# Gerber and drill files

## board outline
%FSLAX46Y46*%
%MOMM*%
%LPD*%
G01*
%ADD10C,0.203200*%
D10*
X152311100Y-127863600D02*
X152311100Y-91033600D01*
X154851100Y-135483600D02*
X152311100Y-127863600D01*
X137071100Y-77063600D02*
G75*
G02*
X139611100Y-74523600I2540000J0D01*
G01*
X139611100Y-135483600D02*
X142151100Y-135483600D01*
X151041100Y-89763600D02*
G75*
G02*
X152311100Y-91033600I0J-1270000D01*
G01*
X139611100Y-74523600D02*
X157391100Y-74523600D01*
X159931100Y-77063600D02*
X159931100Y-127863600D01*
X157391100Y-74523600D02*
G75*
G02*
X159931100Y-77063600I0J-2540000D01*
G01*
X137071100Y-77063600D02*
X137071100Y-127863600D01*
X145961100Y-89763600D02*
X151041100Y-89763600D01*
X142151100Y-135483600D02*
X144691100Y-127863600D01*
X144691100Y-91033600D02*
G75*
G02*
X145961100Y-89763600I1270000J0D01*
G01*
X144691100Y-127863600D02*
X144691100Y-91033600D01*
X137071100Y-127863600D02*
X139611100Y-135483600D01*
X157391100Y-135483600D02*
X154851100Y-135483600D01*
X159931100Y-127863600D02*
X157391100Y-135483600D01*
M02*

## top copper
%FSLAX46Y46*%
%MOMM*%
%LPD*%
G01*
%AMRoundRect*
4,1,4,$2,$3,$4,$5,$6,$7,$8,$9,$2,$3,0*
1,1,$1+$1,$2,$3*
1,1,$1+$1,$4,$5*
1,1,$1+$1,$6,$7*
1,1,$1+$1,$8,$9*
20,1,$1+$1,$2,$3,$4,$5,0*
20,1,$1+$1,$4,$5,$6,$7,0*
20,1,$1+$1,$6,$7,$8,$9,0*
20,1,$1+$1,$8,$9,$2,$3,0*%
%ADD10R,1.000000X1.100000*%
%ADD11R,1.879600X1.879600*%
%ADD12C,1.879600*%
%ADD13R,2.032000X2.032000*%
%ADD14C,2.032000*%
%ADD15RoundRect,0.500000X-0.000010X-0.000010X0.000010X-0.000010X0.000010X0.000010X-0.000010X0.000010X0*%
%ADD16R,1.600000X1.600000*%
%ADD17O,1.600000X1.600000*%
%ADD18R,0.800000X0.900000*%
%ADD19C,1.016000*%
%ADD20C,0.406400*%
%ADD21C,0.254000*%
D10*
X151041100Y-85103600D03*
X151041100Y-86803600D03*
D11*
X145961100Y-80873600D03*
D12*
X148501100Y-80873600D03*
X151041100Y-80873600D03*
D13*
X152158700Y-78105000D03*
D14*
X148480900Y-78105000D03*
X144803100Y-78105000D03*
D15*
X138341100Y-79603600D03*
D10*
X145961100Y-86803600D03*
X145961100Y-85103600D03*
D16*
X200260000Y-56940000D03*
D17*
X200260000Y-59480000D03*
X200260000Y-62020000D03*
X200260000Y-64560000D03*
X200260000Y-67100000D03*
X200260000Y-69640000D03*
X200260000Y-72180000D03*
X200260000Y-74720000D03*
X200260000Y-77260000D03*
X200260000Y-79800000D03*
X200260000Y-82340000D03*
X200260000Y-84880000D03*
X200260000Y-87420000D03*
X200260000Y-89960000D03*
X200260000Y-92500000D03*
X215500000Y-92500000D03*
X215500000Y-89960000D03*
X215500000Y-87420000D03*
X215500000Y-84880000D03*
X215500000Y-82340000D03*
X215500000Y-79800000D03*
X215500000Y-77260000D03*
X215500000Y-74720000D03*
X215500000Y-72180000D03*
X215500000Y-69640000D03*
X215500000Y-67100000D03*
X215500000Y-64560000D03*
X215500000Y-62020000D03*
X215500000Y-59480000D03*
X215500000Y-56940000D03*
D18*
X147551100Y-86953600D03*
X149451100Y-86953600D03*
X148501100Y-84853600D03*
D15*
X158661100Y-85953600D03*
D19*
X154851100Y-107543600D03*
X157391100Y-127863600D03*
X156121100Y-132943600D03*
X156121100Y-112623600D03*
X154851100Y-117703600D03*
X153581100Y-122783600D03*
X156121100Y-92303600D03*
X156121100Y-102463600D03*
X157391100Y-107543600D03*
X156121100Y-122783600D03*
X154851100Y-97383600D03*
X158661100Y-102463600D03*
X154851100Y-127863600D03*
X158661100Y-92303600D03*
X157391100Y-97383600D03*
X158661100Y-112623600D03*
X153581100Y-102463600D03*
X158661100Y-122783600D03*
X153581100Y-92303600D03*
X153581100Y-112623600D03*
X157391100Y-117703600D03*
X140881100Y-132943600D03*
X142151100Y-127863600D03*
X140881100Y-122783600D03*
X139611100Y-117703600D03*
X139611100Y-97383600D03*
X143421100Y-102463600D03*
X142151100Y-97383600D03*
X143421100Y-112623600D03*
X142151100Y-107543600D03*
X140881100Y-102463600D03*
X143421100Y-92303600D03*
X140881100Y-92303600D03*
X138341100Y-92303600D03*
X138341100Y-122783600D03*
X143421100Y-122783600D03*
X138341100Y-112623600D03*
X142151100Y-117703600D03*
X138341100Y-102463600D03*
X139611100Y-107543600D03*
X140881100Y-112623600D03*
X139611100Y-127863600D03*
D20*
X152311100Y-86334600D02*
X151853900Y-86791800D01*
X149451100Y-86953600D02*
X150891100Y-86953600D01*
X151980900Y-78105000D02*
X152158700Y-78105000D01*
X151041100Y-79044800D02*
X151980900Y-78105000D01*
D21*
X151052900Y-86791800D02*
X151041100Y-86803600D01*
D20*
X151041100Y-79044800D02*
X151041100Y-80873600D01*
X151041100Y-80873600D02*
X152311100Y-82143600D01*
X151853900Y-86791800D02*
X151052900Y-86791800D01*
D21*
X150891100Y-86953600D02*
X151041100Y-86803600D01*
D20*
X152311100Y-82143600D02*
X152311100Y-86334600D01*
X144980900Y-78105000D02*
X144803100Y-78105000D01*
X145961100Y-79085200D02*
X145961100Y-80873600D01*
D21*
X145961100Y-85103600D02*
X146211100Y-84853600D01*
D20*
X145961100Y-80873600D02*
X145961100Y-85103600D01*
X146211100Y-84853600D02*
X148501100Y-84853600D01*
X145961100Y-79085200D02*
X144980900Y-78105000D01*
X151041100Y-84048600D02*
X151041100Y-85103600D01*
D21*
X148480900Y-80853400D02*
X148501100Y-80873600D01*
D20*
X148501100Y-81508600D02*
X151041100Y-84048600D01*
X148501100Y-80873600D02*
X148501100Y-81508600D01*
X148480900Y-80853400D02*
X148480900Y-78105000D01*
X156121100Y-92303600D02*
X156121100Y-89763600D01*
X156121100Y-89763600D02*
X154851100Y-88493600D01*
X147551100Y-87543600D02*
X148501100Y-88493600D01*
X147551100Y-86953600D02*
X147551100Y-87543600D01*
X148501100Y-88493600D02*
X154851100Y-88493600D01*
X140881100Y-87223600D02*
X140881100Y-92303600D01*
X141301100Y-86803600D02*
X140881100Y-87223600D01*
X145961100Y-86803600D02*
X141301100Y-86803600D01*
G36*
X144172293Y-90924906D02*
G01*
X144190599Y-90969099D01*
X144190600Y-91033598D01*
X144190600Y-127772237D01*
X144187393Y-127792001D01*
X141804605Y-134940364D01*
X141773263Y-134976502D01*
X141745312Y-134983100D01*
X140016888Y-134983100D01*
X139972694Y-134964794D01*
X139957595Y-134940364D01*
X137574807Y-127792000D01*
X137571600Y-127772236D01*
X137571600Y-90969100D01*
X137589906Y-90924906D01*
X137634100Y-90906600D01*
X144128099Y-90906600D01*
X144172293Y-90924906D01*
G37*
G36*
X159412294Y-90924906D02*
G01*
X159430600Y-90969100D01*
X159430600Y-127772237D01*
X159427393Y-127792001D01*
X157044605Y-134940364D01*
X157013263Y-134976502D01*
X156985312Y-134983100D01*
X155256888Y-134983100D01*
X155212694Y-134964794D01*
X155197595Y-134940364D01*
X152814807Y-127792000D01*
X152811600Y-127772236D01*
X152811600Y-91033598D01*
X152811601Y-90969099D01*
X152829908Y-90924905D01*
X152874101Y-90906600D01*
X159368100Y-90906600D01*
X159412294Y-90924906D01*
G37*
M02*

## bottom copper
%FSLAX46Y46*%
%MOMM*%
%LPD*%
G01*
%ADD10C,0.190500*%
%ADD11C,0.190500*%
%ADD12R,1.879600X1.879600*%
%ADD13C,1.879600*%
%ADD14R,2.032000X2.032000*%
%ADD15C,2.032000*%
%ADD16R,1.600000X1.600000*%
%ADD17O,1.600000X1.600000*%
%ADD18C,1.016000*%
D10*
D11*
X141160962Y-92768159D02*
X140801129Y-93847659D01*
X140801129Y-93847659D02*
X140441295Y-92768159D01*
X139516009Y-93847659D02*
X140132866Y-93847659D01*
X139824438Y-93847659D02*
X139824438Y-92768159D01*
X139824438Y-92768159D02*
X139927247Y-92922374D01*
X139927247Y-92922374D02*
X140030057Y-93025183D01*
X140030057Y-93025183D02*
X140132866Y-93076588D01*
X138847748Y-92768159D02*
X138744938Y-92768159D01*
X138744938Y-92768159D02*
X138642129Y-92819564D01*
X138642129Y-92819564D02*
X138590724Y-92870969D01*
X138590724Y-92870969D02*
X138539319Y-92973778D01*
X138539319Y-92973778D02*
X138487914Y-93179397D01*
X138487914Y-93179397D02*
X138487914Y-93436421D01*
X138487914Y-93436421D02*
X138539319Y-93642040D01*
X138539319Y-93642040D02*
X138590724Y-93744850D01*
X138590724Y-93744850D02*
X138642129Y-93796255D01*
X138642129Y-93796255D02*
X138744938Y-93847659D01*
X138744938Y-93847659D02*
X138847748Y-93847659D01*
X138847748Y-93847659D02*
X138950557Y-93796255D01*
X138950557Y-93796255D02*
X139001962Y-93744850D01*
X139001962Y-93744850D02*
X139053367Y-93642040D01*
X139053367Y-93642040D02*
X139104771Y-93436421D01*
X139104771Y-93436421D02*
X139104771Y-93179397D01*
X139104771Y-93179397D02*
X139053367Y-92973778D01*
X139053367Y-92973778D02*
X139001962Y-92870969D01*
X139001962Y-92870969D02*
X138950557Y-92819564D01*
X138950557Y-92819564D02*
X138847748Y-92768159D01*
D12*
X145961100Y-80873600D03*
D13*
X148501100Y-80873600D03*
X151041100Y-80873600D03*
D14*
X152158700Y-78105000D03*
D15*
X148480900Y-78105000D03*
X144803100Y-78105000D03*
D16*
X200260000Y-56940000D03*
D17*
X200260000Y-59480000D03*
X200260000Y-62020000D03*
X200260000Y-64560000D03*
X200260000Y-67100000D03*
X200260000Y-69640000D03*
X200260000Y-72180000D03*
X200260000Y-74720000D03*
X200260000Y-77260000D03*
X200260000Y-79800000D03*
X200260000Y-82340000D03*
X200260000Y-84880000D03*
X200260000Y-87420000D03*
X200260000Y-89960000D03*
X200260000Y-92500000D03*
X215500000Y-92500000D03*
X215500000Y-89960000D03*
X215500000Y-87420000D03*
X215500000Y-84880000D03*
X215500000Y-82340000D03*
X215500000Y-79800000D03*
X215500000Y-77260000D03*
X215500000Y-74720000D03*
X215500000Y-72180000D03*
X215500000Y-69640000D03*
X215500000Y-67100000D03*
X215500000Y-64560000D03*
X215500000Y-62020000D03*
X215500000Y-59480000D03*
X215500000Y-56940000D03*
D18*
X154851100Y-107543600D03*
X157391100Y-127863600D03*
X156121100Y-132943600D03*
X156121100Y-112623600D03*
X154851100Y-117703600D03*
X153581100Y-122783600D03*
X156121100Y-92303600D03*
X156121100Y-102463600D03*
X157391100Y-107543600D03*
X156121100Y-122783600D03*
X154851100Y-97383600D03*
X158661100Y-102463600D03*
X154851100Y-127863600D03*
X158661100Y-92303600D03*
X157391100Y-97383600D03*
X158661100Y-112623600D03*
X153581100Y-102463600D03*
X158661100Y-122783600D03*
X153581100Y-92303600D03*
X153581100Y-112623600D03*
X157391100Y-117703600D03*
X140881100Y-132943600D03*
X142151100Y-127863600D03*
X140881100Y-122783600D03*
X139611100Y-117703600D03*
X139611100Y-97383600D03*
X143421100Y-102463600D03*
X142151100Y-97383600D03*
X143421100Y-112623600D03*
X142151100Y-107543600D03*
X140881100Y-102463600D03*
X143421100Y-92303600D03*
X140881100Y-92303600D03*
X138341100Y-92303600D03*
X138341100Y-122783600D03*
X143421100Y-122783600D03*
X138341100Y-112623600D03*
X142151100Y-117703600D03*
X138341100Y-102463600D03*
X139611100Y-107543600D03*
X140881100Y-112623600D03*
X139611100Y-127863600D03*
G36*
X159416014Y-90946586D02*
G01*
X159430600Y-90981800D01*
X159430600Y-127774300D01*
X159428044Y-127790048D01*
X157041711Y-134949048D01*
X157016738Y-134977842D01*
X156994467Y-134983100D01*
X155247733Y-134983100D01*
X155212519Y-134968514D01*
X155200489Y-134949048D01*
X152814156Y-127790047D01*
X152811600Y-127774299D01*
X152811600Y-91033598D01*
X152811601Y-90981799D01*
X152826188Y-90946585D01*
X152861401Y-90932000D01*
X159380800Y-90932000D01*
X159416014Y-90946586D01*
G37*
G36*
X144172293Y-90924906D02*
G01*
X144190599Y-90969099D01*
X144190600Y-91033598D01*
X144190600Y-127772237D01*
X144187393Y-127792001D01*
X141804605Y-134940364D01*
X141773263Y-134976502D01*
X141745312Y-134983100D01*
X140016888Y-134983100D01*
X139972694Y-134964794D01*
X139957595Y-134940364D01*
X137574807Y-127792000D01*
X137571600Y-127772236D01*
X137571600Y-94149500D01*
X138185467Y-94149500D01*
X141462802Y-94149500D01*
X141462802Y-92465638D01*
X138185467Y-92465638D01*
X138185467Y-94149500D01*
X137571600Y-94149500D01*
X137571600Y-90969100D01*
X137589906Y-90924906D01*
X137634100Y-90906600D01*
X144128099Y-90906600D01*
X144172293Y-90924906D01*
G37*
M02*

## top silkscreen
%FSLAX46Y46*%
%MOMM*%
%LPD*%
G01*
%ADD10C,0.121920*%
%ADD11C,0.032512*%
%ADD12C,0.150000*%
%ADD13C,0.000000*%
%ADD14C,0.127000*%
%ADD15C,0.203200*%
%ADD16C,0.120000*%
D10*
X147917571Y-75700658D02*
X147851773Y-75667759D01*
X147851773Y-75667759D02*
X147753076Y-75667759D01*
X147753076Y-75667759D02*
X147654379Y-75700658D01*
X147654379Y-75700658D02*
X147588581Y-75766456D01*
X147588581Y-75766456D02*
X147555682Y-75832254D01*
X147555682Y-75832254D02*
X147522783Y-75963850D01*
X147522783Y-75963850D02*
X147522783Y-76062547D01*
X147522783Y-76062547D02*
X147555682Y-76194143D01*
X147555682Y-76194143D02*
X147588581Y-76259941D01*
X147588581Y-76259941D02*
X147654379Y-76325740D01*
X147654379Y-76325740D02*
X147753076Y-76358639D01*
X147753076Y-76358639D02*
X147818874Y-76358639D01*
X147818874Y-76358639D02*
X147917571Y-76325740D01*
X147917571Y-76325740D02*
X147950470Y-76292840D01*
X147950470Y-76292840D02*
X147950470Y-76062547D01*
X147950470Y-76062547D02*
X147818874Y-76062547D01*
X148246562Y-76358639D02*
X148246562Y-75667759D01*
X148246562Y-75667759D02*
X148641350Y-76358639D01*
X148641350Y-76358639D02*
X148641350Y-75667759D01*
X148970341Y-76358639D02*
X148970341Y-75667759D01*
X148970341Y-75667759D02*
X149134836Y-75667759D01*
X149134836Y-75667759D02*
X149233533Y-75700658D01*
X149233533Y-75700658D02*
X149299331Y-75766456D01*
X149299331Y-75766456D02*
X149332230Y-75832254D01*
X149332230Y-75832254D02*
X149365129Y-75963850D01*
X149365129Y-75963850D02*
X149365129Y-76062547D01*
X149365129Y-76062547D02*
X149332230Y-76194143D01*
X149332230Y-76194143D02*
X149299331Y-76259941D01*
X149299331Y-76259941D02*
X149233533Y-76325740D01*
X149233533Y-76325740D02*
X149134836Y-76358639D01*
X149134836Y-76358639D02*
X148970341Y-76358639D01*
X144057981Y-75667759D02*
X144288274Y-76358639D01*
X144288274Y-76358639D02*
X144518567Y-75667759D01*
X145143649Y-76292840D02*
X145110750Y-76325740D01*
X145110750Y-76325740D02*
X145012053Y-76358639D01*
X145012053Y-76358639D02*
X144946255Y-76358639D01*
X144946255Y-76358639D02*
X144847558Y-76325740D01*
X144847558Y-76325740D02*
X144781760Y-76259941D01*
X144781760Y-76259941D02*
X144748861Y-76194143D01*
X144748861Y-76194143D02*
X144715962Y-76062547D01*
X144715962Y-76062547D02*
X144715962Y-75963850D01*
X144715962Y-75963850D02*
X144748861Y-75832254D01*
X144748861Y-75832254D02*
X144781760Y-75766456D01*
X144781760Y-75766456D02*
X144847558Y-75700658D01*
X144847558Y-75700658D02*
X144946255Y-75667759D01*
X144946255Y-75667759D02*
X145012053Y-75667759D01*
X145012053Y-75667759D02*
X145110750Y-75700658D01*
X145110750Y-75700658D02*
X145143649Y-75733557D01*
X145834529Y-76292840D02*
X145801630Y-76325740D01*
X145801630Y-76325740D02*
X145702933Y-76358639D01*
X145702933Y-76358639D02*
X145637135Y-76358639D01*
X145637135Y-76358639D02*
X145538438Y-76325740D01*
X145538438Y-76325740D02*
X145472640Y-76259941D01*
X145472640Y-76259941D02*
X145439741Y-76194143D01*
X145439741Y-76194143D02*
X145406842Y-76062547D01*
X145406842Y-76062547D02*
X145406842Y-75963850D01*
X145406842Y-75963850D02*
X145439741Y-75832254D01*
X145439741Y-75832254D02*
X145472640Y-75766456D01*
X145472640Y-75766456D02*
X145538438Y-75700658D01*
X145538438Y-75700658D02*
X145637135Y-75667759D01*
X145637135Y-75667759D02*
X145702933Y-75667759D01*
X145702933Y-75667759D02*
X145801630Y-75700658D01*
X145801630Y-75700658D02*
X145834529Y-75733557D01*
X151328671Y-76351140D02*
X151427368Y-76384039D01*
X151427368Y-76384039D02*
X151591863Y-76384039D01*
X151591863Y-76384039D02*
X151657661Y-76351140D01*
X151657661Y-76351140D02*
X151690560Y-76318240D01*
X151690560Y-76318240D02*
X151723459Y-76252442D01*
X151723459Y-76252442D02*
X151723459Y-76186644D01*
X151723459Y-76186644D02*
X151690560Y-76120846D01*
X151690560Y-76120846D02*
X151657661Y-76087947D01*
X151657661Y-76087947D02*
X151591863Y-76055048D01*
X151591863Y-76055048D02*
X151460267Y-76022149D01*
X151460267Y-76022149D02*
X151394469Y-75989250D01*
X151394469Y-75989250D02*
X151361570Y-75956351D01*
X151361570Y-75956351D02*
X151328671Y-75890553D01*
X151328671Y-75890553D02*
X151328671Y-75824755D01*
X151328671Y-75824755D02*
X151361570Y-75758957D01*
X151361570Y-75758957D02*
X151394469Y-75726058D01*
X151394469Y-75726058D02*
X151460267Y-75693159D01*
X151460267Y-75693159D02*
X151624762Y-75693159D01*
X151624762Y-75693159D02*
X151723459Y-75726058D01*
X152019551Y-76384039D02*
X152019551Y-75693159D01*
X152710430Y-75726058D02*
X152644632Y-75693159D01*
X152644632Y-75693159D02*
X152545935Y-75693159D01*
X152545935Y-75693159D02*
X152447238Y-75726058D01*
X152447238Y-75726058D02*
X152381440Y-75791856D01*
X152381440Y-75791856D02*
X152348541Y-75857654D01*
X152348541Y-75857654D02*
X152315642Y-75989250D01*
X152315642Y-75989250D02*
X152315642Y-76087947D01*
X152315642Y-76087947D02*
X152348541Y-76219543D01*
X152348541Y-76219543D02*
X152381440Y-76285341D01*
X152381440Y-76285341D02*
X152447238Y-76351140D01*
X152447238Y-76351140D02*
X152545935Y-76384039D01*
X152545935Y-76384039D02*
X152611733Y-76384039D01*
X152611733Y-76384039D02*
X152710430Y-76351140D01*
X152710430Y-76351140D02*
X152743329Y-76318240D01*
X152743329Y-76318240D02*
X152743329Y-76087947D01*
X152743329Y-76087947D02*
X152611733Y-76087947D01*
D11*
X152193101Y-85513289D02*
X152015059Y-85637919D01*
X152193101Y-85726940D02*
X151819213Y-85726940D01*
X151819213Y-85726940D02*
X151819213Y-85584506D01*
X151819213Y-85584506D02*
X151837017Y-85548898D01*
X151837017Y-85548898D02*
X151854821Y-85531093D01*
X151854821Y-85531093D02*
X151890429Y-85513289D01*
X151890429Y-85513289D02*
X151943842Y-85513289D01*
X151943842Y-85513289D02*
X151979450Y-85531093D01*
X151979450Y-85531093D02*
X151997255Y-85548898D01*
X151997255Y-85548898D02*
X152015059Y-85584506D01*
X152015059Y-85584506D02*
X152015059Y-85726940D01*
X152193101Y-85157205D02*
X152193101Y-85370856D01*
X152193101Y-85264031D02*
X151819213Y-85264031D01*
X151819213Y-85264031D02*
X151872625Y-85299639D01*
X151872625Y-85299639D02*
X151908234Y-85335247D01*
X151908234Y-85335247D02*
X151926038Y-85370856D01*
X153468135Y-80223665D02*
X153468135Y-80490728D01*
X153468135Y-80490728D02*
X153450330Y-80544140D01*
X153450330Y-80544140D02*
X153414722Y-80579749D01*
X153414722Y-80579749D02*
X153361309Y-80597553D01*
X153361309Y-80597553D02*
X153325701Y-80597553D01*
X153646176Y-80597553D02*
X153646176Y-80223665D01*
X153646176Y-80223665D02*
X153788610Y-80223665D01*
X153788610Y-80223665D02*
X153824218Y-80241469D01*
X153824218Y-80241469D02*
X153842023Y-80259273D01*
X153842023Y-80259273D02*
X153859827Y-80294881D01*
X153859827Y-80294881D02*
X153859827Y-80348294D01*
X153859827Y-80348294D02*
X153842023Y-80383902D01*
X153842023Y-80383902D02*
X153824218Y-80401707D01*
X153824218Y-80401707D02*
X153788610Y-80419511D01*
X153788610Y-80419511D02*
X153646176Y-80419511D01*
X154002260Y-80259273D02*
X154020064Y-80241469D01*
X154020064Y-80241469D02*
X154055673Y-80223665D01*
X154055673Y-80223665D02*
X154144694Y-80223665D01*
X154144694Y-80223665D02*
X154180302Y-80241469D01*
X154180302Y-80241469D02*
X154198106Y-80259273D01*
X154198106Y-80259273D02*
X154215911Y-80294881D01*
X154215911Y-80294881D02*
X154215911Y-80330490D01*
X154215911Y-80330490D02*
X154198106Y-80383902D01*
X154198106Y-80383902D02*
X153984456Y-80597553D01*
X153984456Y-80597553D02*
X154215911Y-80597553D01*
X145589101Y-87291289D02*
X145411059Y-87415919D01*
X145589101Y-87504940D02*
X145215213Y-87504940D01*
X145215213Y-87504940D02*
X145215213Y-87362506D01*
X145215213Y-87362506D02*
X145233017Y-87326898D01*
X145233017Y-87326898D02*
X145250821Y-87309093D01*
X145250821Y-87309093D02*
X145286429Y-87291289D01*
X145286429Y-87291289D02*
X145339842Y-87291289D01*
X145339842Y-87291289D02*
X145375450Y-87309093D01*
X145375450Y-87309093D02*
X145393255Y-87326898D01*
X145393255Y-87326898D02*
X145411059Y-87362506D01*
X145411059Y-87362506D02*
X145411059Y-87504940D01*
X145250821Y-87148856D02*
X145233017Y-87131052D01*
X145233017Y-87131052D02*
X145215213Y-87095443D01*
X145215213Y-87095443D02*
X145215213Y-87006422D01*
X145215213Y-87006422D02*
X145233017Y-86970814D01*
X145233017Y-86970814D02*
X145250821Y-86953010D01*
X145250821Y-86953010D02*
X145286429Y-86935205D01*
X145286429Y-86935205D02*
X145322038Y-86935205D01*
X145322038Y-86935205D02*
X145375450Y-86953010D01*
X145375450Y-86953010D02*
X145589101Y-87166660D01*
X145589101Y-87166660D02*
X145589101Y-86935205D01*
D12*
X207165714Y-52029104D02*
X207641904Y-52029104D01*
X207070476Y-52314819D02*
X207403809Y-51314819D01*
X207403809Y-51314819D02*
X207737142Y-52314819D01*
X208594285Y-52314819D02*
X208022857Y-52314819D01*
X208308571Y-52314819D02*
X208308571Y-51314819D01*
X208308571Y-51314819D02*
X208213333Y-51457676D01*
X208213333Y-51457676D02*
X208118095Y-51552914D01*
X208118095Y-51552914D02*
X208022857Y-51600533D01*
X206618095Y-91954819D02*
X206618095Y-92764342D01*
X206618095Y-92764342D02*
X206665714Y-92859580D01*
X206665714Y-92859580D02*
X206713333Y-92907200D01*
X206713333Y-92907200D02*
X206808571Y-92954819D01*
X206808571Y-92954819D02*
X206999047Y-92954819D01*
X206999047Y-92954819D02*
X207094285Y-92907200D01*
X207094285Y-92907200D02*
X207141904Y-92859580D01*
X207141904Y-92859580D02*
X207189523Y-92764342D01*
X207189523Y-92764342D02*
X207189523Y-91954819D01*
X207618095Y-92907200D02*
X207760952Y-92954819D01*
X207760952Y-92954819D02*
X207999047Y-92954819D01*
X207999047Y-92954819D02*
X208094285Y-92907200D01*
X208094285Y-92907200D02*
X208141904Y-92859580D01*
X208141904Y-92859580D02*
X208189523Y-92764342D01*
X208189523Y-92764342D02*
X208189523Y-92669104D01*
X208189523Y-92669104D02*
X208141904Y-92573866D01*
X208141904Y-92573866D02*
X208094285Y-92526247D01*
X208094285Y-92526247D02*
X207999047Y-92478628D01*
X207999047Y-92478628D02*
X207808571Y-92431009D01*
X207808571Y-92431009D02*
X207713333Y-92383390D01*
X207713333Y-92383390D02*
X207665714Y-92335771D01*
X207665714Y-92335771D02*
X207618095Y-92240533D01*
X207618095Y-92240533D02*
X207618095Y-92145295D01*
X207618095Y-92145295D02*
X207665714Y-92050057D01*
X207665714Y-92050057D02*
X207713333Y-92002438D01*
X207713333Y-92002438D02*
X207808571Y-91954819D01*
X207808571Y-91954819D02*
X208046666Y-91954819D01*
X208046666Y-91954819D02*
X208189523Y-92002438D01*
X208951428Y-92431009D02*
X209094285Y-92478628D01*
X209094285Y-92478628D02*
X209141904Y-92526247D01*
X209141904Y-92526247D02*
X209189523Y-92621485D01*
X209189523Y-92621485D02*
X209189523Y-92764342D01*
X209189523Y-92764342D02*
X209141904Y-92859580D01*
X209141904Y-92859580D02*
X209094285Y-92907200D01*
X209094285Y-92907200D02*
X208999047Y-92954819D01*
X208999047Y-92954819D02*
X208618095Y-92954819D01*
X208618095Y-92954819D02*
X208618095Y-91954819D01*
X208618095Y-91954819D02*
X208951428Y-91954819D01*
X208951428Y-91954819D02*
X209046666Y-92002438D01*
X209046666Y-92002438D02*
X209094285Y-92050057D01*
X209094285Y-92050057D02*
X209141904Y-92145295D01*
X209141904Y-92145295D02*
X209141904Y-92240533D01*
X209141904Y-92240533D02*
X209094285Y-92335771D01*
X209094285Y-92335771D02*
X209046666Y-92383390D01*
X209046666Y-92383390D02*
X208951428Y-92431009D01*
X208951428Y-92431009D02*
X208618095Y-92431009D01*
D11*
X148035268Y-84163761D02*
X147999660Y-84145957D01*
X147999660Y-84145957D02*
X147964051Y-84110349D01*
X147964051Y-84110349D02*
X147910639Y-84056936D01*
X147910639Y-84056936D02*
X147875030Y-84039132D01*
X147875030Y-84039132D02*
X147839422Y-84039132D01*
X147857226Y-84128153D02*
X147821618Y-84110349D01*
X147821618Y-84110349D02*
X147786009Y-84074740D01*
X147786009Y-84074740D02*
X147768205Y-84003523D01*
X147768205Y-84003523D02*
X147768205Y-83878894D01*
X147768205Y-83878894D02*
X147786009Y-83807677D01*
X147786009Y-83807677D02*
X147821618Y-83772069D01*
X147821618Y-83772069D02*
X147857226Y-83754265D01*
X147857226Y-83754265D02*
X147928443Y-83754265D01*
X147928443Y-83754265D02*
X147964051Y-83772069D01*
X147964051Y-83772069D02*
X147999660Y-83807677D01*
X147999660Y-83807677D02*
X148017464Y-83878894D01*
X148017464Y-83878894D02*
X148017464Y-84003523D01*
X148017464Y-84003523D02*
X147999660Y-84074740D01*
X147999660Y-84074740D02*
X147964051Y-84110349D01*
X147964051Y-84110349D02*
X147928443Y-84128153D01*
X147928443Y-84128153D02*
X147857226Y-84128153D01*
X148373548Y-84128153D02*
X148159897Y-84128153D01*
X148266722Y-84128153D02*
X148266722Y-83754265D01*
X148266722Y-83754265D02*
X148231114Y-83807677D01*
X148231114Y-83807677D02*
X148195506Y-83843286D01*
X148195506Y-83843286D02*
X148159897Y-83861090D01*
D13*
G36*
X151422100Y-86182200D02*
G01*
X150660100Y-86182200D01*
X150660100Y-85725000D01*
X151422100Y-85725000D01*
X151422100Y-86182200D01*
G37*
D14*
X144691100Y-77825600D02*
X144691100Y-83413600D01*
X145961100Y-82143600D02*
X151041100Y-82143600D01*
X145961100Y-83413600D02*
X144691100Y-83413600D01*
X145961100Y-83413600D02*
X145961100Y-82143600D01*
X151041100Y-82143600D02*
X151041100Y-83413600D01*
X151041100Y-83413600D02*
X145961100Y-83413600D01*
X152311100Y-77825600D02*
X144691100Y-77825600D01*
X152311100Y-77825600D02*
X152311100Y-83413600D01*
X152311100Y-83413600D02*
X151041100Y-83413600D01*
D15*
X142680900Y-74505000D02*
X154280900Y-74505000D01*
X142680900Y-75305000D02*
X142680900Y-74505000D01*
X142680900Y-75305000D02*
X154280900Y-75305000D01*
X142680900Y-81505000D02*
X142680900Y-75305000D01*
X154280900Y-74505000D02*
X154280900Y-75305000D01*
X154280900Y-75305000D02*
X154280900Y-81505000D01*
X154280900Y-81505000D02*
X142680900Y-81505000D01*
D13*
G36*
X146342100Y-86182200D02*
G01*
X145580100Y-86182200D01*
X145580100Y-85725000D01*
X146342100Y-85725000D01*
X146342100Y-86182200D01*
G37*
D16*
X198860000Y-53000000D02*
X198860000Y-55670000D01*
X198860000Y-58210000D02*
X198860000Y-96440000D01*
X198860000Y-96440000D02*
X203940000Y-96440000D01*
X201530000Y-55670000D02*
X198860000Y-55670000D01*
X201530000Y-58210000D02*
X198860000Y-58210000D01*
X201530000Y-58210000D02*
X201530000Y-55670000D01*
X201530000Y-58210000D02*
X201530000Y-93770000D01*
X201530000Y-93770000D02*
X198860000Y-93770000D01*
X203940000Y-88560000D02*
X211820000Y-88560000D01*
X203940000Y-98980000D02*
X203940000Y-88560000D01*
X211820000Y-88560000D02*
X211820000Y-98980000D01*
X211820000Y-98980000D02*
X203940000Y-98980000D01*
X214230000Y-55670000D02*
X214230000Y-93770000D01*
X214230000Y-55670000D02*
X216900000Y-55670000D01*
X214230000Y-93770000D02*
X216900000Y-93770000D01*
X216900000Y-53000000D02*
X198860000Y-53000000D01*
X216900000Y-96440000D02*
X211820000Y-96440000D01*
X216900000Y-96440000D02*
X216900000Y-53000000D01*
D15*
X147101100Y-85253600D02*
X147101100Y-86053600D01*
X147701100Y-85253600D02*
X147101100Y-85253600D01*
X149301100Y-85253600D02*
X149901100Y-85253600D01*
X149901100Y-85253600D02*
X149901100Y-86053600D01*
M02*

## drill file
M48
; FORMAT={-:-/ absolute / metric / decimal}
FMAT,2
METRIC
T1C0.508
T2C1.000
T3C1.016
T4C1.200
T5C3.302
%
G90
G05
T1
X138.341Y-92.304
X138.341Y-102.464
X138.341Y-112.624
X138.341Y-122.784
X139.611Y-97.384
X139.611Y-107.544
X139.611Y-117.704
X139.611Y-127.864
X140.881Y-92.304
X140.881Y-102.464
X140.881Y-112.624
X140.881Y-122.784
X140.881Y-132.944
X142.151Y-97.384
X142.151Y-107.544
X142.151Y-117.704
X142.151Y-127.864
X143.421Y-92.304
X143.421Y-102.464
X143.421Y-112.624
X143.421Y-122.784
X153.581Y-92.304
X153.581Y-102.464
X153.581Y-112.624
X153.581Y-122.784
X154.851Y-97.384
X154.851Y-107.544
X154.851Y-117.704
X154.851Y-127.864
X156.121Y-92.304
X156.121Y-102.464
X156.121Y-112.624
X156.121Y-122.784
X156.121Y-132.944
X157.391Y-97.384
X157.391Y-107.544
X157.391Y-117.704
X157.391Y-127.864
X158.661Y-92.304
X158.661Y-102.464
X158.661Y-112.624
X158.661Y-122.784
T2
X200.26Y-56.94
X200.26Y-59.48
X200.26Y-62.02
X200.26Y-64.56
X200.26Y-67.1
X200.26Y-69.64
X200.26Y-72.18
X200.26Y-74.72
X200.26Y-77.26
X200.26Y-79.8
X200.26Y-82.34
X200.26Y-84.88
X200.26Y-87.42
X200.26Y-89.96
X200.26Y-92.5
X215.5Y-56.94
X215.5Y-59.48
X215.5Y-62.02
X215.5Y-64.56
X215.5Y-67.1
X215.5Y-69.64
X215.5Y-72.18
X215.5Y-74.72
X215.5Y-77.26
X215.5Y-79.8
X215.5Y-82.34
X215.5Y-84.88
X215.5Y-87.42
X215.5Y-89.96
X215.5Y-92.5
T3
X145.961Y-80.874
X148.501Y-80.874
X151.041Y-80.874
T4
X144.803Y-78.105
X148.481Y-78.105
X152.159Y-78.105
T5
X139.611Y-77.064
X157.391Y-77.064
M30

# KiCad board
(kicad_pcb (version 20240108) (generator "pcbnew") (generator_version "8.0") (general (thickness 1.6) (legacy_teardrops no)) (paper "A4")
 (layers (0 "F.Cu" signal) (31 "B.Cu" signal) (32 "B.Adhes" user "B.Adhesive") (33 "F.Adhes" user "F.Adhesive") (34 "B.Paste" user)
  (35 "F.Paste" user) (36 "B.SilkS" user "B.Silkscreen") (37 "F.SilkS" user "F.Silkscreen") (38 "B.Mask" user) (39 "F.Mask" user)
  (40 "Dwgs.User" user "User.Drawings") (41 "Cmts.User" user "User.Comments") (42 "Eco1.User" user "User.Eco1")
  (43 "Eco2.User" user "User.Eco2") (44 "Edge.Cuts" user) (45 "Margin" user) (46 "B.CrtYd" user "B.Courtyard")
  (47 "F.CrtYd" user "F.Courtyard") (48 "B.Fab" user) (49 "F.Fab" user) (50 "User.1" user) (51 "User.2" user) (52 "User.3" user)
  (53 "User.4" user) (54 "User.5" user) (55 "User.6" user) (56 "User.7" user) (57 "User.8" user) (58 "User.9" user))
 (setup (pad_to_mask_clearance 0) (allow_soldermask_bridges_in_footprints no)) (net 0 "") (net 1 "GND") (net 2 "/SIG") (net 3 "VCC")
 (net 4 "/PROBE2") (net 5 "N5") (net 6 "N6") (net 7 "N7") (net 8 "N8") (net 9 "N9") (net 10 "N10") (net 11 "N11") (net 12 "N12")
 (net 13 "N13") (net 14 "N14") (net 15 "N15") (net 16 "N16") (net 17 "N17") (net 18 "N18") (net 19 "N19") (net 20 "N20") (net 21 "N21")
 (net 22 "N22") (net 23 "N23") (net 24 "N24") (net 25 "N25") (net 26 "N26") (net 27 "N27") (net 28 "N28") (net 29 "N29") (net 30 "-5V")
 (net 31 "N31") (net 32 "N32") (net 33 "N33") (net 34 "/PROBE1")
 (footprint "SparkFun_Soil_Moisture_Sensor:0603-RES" (layer "F.Cu") (at 151.0411 85.9536 -90)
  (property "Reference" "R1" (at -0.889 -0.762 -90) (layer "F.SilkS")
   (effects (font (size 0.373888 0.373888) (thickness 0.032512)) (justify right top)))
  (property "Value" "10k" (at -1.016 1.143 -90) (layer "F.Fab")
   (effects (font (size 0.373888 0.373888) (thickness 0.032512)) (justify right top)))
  (fp_poly
   (pts (xy -0.2286 0.381) (xy 0.2286 0.381) (xy 0.2286 -0.381) (xy -0.2286 -0.381)) (stroke (width 0) (type default)) (fill solid)
   (layer "F.SilkS"))
  (pad "1" smd rect (at -0.85 0 270) (size 1.1 1) (layers "F.Cu" "F.Paste" "F.Mask") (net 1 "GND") (solder_mask_margin 0.1016)
   (thermal_bridge_angle 0))
  (pad "2" smd rect (at 0.85 0 270) (size 1.1 1) (layers "F.Cu" "F.Paste" "F.Mask") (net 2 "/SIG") (solder_mask_margin 0.1016)
   (thermal_bridge_angle 0)))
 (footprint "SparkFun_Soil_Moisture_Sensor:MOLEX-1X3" (layer "F.Cu") (at 145.9611 80.8736)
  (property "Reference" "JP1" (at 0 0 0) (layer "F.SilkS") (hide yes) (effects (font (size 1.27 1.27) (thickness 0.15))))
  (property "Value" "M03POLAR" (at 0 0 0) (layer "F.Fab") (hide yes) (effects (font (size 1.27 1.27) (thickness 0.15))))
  (fp_line (start -1.27 -3.048) (end -1.27 2.54) (stroke (width 0.127) (type solid)) (layer "F.SilkS"))
  (fp_line (start 0 1.27) (end 5.08 1.27) (stroke (width 0.127) (type solid)) (layer "F.SilkS"))
  (fp_line (start 0 2.54) (end -1.27 2.54) (stroke (width 0.127) (type solid)) (layer "F.SilkS"))
  (fp_line (start 0 2.54) (end 0 1.27) (stroke (width 0.127) (type solid)) (layer "F.SilkS"))
  (fp_line (start 5.08 1.27) (end 5.08 2.54) (stroke (width 0.127) (type solid)) (layer "F.SilkS"))
  (fp_line (start 5.08 2.54) (end 0 2.54) (stroke (width 0.127) (type solid)) (layer "F.SilkS"))
  (fp_line (start 6.35 -3.048) (end -1.27 -3.048) (stroke (width 0.127) (type solid)) (layer "F.SilkS"))
  (fp_line (start 6.35 -3.048) (end 6.35 2.54) (stroke (width 0.127) (type solid)) (layer "F.SilkS"))
  (fp_line (start 6.35 2.54) (end 5.08 2.54) (stroke (width 0.127) (type solid)) (layer "F.SilkS"))
  (pad "1" thru_hole rect (at 0 0) (size 1.8796 1.8796) (drill 1.016) (layers "*.Cu" "*.Mask") (remove_unused_layers no) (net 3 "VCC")
   (solder_mask_margin 0.1016) (thermal_bridge_angle 0))
  (pad "2" thru_hole circle (at 2.54 0) (size 1.8796 1.8796) (drill 1.016) (layers "*.Cu" "*.Mask") (remove_unused_layers no) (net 1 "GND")
   (solder_mask_margin 0.1016) (thermal_bridge_angle 0))
  (pad "3" thru_hole circle (at 5.08 0) (size 1.8796 1.8796) (drill 1.016) (layers "*.Cu" "*.Mask") (remove_unused_layers no) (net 2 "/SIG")
   (solder_mask_margin 0.1016) (thermal_bridge_angle 0)))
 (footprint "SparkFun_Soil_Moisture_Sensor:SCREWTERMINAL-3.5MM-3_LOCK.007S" (layer "F.Cu") (at 151.9809 78.105 180)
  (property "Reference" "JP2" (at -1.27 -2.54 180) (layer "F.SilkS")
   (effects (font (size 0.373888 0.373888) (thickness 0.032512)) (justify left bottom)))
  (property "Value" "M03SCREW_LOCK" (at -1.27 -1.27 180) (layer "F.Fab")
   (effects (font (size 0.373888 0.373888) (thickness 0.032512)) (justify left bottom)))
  (fp_line (start 9.3 3.6) (end -2.3 3.6) (stroke (width 0.2032) (type solid)) (layer "F.SilkS"))
  (fp_line (start 9.3 2.8) (end 9.3 3.6) (stroke (width 0.2032) (type solid)) (layer "F.SilkS"))
  (fp_line (start 9.3 2.8) (end -2.3 2.8) (stroke (width 0.2032) (type solid)) (layer "F.SilkS"))
  (fp_line (start 9.3 -3.4) (end 9.3 2.8) (stroke (width 0.2032) (type solid)) (layer "F.SilkS"))
  (fp_line (start -2.3 3.6) (end -2.3 2.8) (stroke (width 0.2032) (type solid)) (layer "F.SilkS"))
  (fp_line (start -2.3 2.8) (end -2.3 -3.4) (stroke (width 0.2032) (type solid)) (layer "F.SilkS"))
  (fp_line (start -2.3 -3.4) (end 9.3 -3.4) (stroke (width 0.2032) (type solid)) (layer "F.SilkS"))
  (pad "1" thru_hole rect (at -0.1778 0 180) (size 2.032 2.032) (drill 1.2) (layers "*.Cu" "*.Mask") (remove_unused_layers no)
   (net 2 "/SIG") (solder_mask_margin 0.1016) (thermal_bridge_angle 0))
  (pad "2" thru_hole circle (at 3.5 0 180) (size 2.032 2.032) (drill 1.2) (layers "*.Cu" "*.Mask") (remove_unused_layers no) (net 1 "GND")
   (solder_mask_margin 0.1016) (thermal_bridge_angle 0))
  (pad "3" thru_hole circle (at 7.1778 0 180) (size 2.032 2.032) (drill 1.2) (layers "*.Cu" "*.Mask") (remove_unused_layers no)
   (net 3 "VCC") (solder_mask_margin 0.1016) (thermal_bridge_angle 0)))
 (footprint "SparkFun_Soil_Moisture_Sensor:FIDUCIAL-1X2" (layer "F.Cu") (at 138.3411 79.6036)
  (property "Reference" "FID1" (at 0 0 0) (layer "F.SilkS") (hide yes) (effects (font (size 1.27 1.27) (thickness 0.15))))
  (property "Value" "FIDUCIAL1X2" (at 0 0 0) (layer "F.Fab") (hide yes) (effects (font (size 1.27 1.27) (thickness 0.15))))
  (pad "1" smd roundrect (at 0 0) (size 1 1) (layers "F.Cu" "F.Mask") (roundrect_rratio 0.5) (solder_mask_margin 0.1016)
   (thermal_bridge_angle 0)))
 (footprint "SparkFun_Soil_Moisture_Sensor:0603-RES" (layer "F.Cu") (at 145.9611 85.9536 90)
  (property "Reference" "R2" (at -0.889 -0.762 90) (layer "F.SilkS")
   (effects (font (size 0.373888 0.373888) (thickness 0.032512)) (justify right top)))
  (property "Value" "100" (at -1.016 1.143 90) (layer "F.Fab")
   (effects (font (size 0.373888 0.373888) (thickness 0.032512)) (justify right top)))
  (fp_poly
   (pts (xy -0.2286 0.381) (xy 0.2286 0.381) (xy 0.2286 -0.381) (xy -0.2286 -0.381)) (stroke (width 0) (type default)) (fill solid)
   (layer "F.SilkS"))
  (pad "1" smd rect (at -0.85 0 90) (size 1.1 1) (layers "F.Cu" "F.Paste" "F.Mask") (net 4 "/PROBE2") (solder_mask_margin 0.1016)
   (thermal_bridge_angle 0))
  (pad "2" smd rect (at 0.85 0 90) (size 1.1 1) (layers "F.Cu" "F.Paste" "F.Mask") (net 3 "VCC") (solder_mask_margin 0.1016)
   (thermal_bridge_angle 0)))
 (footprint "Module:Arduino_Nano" (layer "F.Cu") (at 200.26 56.94)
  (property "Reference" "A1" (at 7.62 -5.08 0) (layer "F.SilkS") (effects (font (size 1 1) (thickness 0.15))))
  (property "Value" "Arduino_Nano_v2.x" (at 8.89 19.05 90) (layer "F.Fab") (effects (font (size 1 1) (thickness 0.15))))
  (fp_line (start -1.4 -3.94) (end -1.4 -1.27) (stroke (width 0.12) (type solid)) (layer "F.SilkS"))
  (fp_line (start -1.4 1.27) (end -1.4 39.5) (stroke (width 0.12) (type solid)) (layer "F.SilkS"))
  (fp_line (start -1.4 39.5) (end 3.68 39.5) (stroke (width 0.12) (type solid)) (layer "F.SilkS"))
  (fp_line (start 1.27 -1.27) (end -1.4 -1.27) (stroke (width 0.12) (type solid)) (layer "F.SilkS"))
  (fp_line (start 1.27 1.27) (end -1.4 1.27) (stroke (width 0.12) (type solid)) (layer "F.SilkS"))
  (fp_line (start 1.27 1.27) (end 1.27 -1.27) (stroke (width 0.12) (type solid)) (layer "F.SilkS"))
  (fp_line (start 1.27 1.27) (end 1.27 36.83) (stroke (width 0.12) (type solid)) (layer "F.SilkS"))
  (fp_line (start 1.27 36.83) (end -1.4 36.83) (stroke (width 0.12) (type solid)) (layer "F.SilkS"))
  (fp_line (start 3.68 31.62) (end 11.56 31.62) (stroke (width 0.12) (type solid)) (layer "F.SilkS"))
  (fp_line (start 3.68 42.04) (end 3.68 31.62) (stroke (width 0.12) (type solid)) (layer "F.SilkS"))
  (fp_line (start 11.56 31.62) (end 11.56 42.04) (stroke (width 0.12) (type solid)) (layer "F.SilkS"))
  (fp_line (start 11.56 42.04) (end 3.68 42.04) (stroke (width 0.12) (type solid)) (layer "F.SilkS"))
  (fp_line (start 13.97 -1.27) (end 13.97 36.83) (stroke (width 0.12) (type solid)) (layer "F.SilkS"))
  (fp_line (start 13.97 -1.27) (end 16.64 -1.27) (stroke (width 0.12) (type solid)) (layer "F.SilkS"))
  (fp_line (start 13.97 36.83) (end 16.64 36.83) (stroke (width 0.12) (type solid)) (layer "F.SilkS"))
  (fp_line (start 16.64 -3.94) (end -1.4 -3.94) (stroke (width 0.12) (type solid)) (layer "F.SilkS"))
  (fp_line (start 16.64 39.5) (end 11.56 39.5) (stroke (width 0.12) (type solid)) (layer "F.SilkS"))
  (fp_line (start 16.64 39.5) (end 16.64 -3.94) (stroke (width 0.12) (type solid)) (layer "F.SilkS"))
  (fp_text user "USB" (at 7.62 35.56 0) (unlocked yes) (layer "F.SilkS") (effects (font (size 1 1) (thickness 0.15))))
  (pad "1" thru_hole rect (at 0 0) (size 1.6 1.6) (drill 1) (layers "*.Cu" "*.Mask") (remove_unused_layers no) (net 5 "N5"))
  (pad "2" thru_hole oval (at 0 2.54) (size 1.6 1.6) (drill 1) (layers "*.Cu" "*.Mask") (remove_unused_layers no) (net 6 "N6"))
  (pad "3" thru_hole oval (at 0 5.08) (size 1.6 1.6) (drill 1) (layers "*.Cu" "*.Mask") (remove_unused_layers no) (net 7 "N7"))
  (pad "4" thru_hole oval (at 0 7.62) (size 1.6 1.6) (drill 1) (layers "*.Cu" "*.Mask") (remove_unused_layers no) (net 1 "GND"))
  (pad "5" thru_hole oval (at 0 10.16) (size 1.6 1.6) (drill 1) (layers "*.Cu" "*.Mask") (remove_unused_layers no) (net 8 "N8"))
  (pad "6" thru_hole oval (at 0 12.7) (size 1.6 1.6) (drill 1) (layers "*.Cu" "*.Mask") (remove_unused_layers no) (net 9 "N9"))
  (pad "7" thru_hole oval (at 0 15.24) (size 1.6 1.6) (drill 1) (layers "*.Cu" "*.Mask") (remove_unused_layers no) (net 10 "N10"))
  (pad "8" thru_hole oval (at 0 17.78) (size 1.6 1.6) (drill 1) (layers "*.Cu" "*.Mask") (remove_unused_layers no) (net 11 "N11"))
  (pad "9" thru_hole oval (at 0 20.32) (size 1.6 1.6) (drill 1) (layers "*.Cu" "*.Mask") (remove_unused_layers no) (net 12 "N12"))
  (pad "10" thru_hole oval (at 0 22.86) (size 1.6 1.6) (drill 1) (layers "*.Cu" "*.Mask") (remove_unused_layers no) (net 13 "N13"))
  (pad "11" thru_hole oval (at 0 25.4) (size 1.6 1.6) (drill 1) (layers "*.Cu" "*.Mask") (remove_unused_layers no) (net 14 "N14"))
  (pad "12" thru_hole oval (at 0 27.94) (size 1.6 1.6) (drill 1) (layers "*.Cu" "*.Mask") (remove_unused_layers no) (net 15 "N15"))
  (pad "13" thru_hole oval (at 0 30.48) (size 1.6 1.6) (drill 1) (layers "*.Cu" "*.Mask") (remove_unused_layers no) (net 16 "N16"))
  (pad "14" thru_hole oval (at 0 33.02) (size 1.6 1.6) (drill 1) (layers "*.Cu" "*.Mask") (remove_unused_layers no) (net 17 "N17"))
  (pad "15" thru_hole oval (at 0 35.56) (size 1.6 1.6) (drill 1) (layers "*.Cu" "*.Mask") (remove_unused_layers no) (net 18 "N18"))
  (pad "16" thru_hole oval (at 15.24 35.56) (size 1.6 1.6) (drill 1) (layers "*.Cu" "*.Mask") (remove_unused_layers no) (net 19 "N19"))
  (pad "17" thru_hole oval (at 15.24 33.02) (size 1.6 1.6) (drill 1) (layers "*.Cu" "*.Mask") (remove_unused_layers no) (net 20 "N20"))
  (pad "18" thru_hole oval (at 15.24 30.48) (size 1.6 1.6) (drill 1) (layers "*.Cu" "*.Mask") (remove_unused_layers no) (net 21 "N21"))
  (pad "19" thru_hole oval (at 15.24 27.94) (size 1.6 1.6) (drill 1) (layers "*.Cu" "*.Mask") (remove_unused_layers no) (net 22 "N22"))
  (pad "20" thru_hole oval (at 15.24 25.4) (size 1.6 1.6) (drill 1) (layers "*.Cu" "*.Mask") (remove_unused_layers no) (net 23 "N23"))
  (pad "21" thru_hole oval (at 15.24 22.86) (size 1.6 1.6) (drill 1) (layers "*.Cu" "*.Mask") (remove_unused_layers no) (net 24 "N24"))
  (pad "22" thru_hole oval (at 15.24 20.32) (size 1.6 1.6) (drill 1) (layers "*.Cu" "*.Mask") (remove_unused_layers no) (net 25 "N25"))
  (pad "23" thru_hole oval (at 15.24 17.78) (size 1.6 1.6) (drill 1) (layers "*.Cu" "*.Mask") (remove_unused_layers no) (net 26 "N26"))
  (pad "24" thru_hole oval (at 15.24 15.24) (size 1.6 1.6) (drill 1) (layers "*.Cu" "*.Mask") (remove_unused_layers no) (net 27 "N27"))
  (pad "25" thru_hole oval (at 15.24 12.7) (size 1.6 1.6) (drill 1) (layers "*.Cu" "*.Mask") (remove_unused_layers no) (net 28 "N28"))
  (pad "26" thru_hole oval (at 15.24 10.16) (size 1.6 1.6) (drill 1) (layers "*.Cu" "*.Mask") (remove_unused_layers no) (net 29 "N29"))
  (pad "27" thru_hole oval (at 15.24 7.62) (size 1.6 1.6) (drill 1) (layers "*.Cu" "*.Mask") (remove_unused_layers no) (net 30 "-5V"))
  (pad "28" thru_hole oval (at 15.24 5.08) (size 1.6 1.6) (drill 1) (layers "*.Cu" "*.Mask") (remove_unused_layers no) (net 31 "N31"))
  (pad "29" thru_hole oval (at 15.24 2.54) (size 1.6 1.6) (drill 1) (layers "*.Cu" "*.Mask") (remove_unused_layers no) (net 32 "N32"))
  (pad "30" thru_hole oval (at 15.24 0) (size 1.6 1.6) (drill 1) (layers "*.Cu" "*.Mask") (remove_unused_layers no) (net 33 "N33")))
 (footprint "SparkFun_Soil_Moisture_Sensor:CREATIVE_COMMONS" (layer "F.Cu") (at 129.4511 145.6436)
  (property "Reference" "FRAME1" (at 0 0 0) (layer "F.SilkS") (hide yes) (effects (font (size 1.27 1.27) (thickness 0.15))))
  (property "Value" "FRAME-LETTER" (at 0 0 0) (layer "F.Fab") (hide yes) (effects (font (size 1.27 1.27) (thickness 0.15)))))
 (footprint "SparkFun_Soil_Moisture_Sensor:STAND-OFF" (layer "F.Cu") (at 139.6111 77.0636)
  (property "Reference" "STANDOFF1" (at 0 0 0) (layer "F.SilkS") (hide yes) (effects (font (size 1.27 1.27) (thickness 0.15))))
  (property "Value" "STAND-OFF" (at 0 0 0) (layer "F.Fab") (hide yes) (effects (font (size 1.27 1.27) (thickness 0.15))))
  (pad "" np_thru_hole circle (at 0 0) (size 3.302 3.302) (drill 3.302) (layers "*.Cu" "*.Mask")))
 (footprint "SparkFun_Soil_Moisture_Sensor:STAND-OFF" (layer "F.Cu") (at 157.3911 77.0636)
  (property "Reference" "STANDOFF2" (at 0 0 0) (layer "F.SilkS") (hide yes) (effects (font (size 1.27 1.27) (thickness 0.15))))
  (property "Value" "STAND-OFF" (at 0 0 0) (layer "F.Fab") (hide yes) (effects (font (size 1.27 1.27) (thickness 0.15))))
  (pad "" np_thru_hole circle (at 0 0) (size 3.302 3.302) (drill 3.302) (layers "*.Cu" "*.Mask")))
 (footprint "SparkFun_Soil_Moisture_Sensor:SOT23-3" (layer "F.Cu") (at 148.5011 85.9536)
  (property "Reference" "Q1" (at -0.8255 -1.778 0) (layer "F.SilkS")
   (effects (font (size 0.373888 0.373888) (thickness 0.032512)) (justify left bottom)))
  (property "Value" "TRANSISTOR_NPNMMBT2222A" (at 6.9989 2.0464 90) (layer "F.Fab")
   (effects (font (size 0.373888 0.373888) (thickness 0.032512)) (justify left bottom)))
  (fp_line (start -1.4 -0.7) (end -1.4 0.1) (stroke (width 0.2032) (type solid)) (layer "F.SilkS"))
  (fp_line (start -0.8 -0.7) (end -1.4 -0.7) (stroke (width 0.2032) (type solid)) (layer "F.SilkS"))
  (fp_line (start 0.8 -0.7) (end 1.4 -0.7) (stroke (width 0.2032) (type solid)) (layer "F.SilkS"))
  (fp_line (start 1.4 -0.7) (end 1.4 0.1) (stroke (width 0.2032) (type solid)) (layer "F.SilkS"))
  (pad "1" smd rect (at -0.95 1) (size 0.8 0.9) (layers "F.Cu" "F.Paste" "F.Mask") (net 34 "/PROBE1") (solder_mask_margin 0.1016)
   (thermal_bridge_angle 0))
  (pad "2" smd rect (at 0.95 1) (size 0.8 0.9) (layers "F.Cu" "F.Paste" "F.Mask") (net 2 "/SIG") (solder_mask_margin 0.1016)
   (thermal_bridge_angle 0))
  (pad "3" smd rect (at 0 -1.1) (size 0.8 0.9) (layers "F.Cu" "F.Paste" "F.Mask") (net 3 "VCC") (solder_mask_margin 0.1016)
   (thermal_bridge_angle 0)))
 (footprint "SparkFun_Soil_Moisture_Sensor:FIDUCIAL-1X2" (layer "F.Cu") (at 158.6611 85.9536)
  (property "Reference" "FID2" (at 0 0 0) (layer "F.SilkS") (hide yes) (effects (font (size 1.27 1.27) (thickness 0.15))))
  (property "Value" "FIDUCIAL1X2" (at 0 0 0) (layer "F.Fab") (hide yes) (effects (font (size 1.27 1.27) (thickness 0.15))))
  (pad "1" smd roundrect (at 0 0) (size 1 1) (layers "F.Cu" "F.Mask") (roundrect_rratio 0.5) (solder_mask_margin 0.1016)
   (thermal_bridge_angle 0)))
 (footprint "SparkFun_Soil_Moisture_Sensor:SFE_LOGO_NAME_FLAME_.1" (layer "B.Cu") (at 154.8511 87.2236 180)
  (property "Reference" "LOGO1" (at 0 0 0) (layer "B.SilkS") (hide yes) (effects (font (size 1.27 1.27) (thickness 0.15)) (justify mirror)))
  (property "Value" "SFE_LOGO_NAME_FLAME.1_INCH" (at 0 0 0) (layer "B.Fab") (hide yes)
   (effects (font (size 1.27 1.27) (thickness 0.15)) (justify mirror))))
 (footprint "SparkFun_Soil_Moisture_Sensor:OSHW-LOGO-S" (layer "B.Cu") (at 157.3911 80.8736 180)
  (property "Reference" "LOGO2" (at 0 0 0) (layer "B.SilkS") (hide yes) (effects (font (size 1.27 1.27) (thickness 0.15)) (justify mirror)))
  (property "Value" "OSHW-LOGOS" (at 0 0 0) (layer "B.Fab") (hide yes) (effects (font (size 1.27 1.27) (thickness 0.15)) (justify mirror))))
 (gr_line (start 152.3111 127.8636) (end 152.3111 91.0336) (stroke (width 0.2032) (type solid)) (layer "Edge.Cuts"))
 (gr_line (start 154.8511 135.4836) (end 152.3111 127.8636) (stroke (width 0.2032) (type solid)) (layer "Edge.Cuts"))
 (gr_arc (start 137.0711 77.0636) (mid 137.815049 75.267549) (end 139.6111 74.5236) (stroke (width 0.2032) (type solid)) (layer "Edge.Cuts"))
 (gr_line (start 139.6111 135.4836) (end 142.1511 135.4836) (stroke (width 0.2032) (type solid)) (layer "Edge.Cuts"))
 (gr_arc (start 151.0411 89.7636) (mid 151.939126 90.135574) (end 152.3111 91.0336) (stroke (width 0.2032) (type solid)) (layer "Edge.Cuts"))
 (gr_line (start 139.6111 74.5236) (end 157.3911 74.5236) (stroke (width 0.2032) (type solid)) (layer "Edge.Cuts"))
 (gr_line (start 159.9311 77.0636) (end 159.9311 127.8636) (stroke (width 0.2032) (type solid)) (layer "Edge.Cuts"))
 (gr_arc (start 157.3911 74.5236) (mid 159.187151 75.267549) (end 159.9311 77.0636) (stroke (width 0.2032) (type solid)) (layer "Edge.Cuts"))
 (gr_line (start 137.0711 77.0636) (end 137.0711 127.8636) (stroke (width 0.2032) (type solid)) (layer "Edge.Cuts"))
 (gr_line (start 145.9611 89.7636) (end 151.0411 89.7636) (stroke (width 0.2032) (type solid)) (layer "Edge.Cuts"))
 (gr_line (start 142.1511 135.4836) (end 144.6911 127.8636) (stroke (width 0.2032) (type solid)) (layer "Edge.Cuts"))
 (gr_arc (start 144.6911 91.0336) (mid 145.063074 90.135574) (end 145.9611 89.7636) (stroke (width 0.2032) (type solid)) (layer "Edge.Cuts"))
 (gr_line (start 144.6911 127.8636) (end 144.6911 91.0336) (stroke (width 0.2032) (type solid)) (layer "Edge.Cuts"))
 (gr_line (start 137.0711 127.8636) (end 139.6111 135.4836) (stroke (width 0.2032) (type solid)) (layer "Edge.Cuts"))
 (gr_line (start 157.3911 135.4836) (end 154.8511 135.4836) (stroke (width 0.2032) (type solid)) (layer "Edge.Cuts"))
 (gr_line (start 159.9311 127.8636) (end 157.3911 135.4836) (stroke (width 0.2032) (type solid)) (layer "Edge.Cuts"))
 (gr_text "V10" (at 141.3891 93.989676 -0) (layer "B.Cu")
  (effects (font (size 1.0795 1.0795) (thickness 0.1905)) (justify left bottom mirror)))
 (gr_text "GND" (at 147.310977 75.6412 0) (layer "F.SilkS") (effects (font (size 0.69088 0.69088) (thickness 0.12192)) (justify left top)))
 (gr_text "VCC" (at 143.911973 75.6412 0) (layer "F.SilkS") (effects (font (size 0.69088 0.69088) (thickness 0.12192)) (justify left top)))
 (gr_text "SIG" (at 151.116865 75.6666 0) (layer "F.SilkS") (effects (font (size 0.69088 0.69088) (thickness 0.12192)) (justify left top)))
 (segment (start 152.3111 86.3346) (end 151.8539 86.7918) (width 0.4064) (layer "F.Cu") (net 2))
 (segment (start 149.4511 86.9536) (end 150.8911 86.9536) (width 0.4064) (layer "F.Cu") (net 2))
 (segment (start 151.9809 78.105) (end 152.1587 78.105) (width 0.4064) (layer "F.Cu") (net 2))
 (segment (start 151.0411 79.0448) (end 151.9809 78.105) (width 0.4064) (layer "F.Cu") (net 2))
 (segment (start 151.0529 86.7918) (end 151.0411 86.8036) (width 0.254) (layer "F.Cu") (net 2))
 (segment (start 151.0411 79.0448) (end 151.0411 80.8736) (width 0.4064) (layer "F.Cu") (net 2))
 (segment (start 151.0411 80.8736) (end 152.3111 82.1436) (width 0.4064) (layer "F.Cu") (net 2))
 (segment (start 151.8539 86.7918) (end 151.0529 86.7918) (width 0.4064) (layer "F.Cu") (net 2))
 (segment (start 150.8911 86.9536) (end 151.0411 86.8036) (width 0.254) (layer "F.Cu") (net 2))
 (segment (start 152.3111 82.1436) (end 152.3111 86.3346) (width 0.4064) (layer "F.Cu") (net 2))
 (segment (start 144.9809 78.105) (end 144.8031 78.105) (width 0.4064) (layer "F.Cu") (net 3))
 (segment (start 145.9611 79.0852) (end 145.9611 80.8736) (width 0.4064) (layer "F.Cu") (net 3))
 (segment (start 145.9611 85.1036) (end 146.2111 84.8536) (width 0.254) (layer "F.Cu") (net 3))
 (segment (start 145.9611 80.8736) (end 145.9611 85.1036) (width 0.4064) (layer "F.Cu") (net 3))
 (segment (start 146.2111 84.8536) (end 148.5011 84.8536) (width 0.4064) (layer "F.Cu") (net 3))
 (segment (start 145.9611 79.0852) (end 144.9809 78.105) (width 0.4064) (layer "F.Cu") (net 3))
 (segment (start 151.0411 84.0486) (end 151.0411 85.1036) (width 0.4064) (layer "F.Cu") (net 1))
 (segment (start 148.4809 80.8534) (end 148.5011 80.8736) (width 0.254) (layer "F.Cu") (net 1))
 (segment (start 148.5011 81.5086) (end 151.0411 84.0486) (width 0.4064) (layer "F.Cu") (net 1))
 (segment (start 148.5011 80.8736) (end 148.5011 81.5086) (width 0.4064) (layer "F.Cu") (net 1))
 (segment (start 148.4809 80.8534) (end 148.4809 78.105) (width 0.4064) (layer "F.Cu") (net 1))
 (segment (start 156.1211 92.3036) (end 156.1211 89.7636) (width 0.4064) (layer "F.Cu") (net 34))
 (segment (start 156.1211 89.7636) (end 154.8511 88.4936) (width 0.4064) (layer "F.Cu") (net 34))
 (segment (start 147.5511 87.5436) (end 148.5011 88.4936) (width 0.4064) (layer "F.Cu") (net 34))
 (segment (start 147.5511 86.9536) (end 147.5511 87.5436) (width 0.4064) (layer "F.Cu") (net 34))
 (segment (start 148.5011 88.4936) (end 154.8511 88.4936) (width 0.4064) (layer "F.Cu") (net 34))
 (via (at 154.8511 107.5436) (size 1.016) (drill 0.508) (layers "F.Cu" "B.Cu") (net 34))
 (via (at 157.3911 127.8636) (size 1.016) (drill 0.508) (layers "F.Cu" "B.Cu") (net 34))
 (via (at 156.1211 132.9436) (size 1.016) (drill 0.508) (layers "F.Cu" "B.Cu") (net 34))
 (via (at 156.1211 112.6236) (size 1.016) (drill 0.508) (layers "F.Cu" "B.Cu") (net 34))
 (via (at 154.8511 117.7036) (size 1.016) (drill 0.508) (layers "F.Cu" "B.Cu") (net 34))
 (via (at 153.5811 122.7836) (size 1.016) (drill 0.508) (layers "F.Cu" "B.Cu") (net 34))
 (via (at 156.1211 92.3036) (size 1.016) (drill 0.508) (layers "F.Cu" "B.Cu") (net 34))
 (via (at 156.1211 102.4636) (size 1.016) (drill 0.508) (layers "F.Cu" "B.Cu") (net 34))
 (via (at 157.3911 107.5436) (size 1.016) (drill 0.508) (layers "F.Cu" "B.Cu") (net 34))
 (via (at 156.1211 122.7836) (size 1.016) (drill 0.508) (layers "F.Cu" "B.Cu") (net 34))
 (via (at 154.8511 97.3836) (size 1.016) (drill 0.508) (layers "F.Cu" "B.Cu") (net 34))
 (via (at 158.6611 102.4636) (size 1.016) (drill 0.508) (layers "F.Cu" "B.Cu") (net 34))
 (via (at 154.8511 127.8636) (size 1.016) (drill 0.508) (layers "F.Cu" "B.Cu") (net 34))
 (via (at 158.6611 92.3036) (size 1.016) (drill 0.508) (layers "F.Cu" "B.Cu") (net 34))
 (via (at 157.3911 97.3836) (size 1.016) (drill 0.508) (layers "F.Cu" "B.Cu") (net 34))
 (via (at 158.6611 112.6236) (size 1.016) (drill 0.508) (layers "F.Cu" "B.Cu") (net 34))
 (via (at 153.5811 102.4636) (size 1.016) (drill 0.508) (layers "F.Cu" "B.Cu") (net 34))
 (via (at 158.6611 122.7836) (size 1.016) (drill 0.508) (layers "F.Cu" "B.Cu") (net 34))
 (via (at 153.5811 92.3036) (size 1.016) (drill 0.508) (layers "F.Cu" "B.Cu") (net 34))
 (via (at 153.5811 112.6236) (size 1.016) (drill 0.508) (layers "F.Cu" "B.Cu") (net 34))
 (via (at 157.3911 117.7036) (size 1.016) (drill 0.508) (layers "F.Cu" "B.Cu") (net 34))
 (segment (start 140.8811 87.2236) (end 140.8811 92.3036) (width 0.4064) (layer "F.Cu") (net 4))
 (segment (start 141.3011 86.8036) (end 140.8811 87.2236) (width 0.4064) (layer "F.Cu") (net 4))
 (segment (start 145.9611 86.8036) (end 141.3011 86.8036) (width 0.4064) (layer "F.Cu") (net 4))
 (via (at 140.8811 132.9436) (size 1.016) (drill 0.508) (layers "F.Cu" "B.Cu") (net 4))
 (via (at 142.1511 127.8636) (size 1.016) (drill 0.508) (layers "F.Cu" "B.Cu") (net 4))
 (via (at 140.8811 122.7836) (size 1.016) (drill 0.508) (layers "F.Cu" "B.Cu") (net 4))
 (via (at 139.6111 117.7036) (size 1.016) (drill 0.508) (layers "F.Cu" "B.Cu") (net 4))
 (via (at 139.6111 97.3836) (size 1.016) (drill 0.508) (layers "F.Cu" "B.Cu") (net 4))
 (via (at 143.4211 102.4636) (size 1.016) (drill 0.508) (layers "F.Cu" "B.Cu") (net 4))
 (via (at 142.1511 97.3836) (size 1.016) (drill 0.508) (layers "F.Cu" "B.Cu") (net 4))
 (via (at 143.4211 112.6236) (size 1.016) (drill 0.508) (layers "F.Cu" "B.Cu") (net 4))
 (via (at 142.1511 107.5436) (size 1.016) (drill 0.508) (layers "F.Cu" "B.Cu") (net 4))
 (via (at 140.8811 102.4636) (size 1.016) (drill 0.508) (layers "F.Cu" "B.Cu") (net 4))
 (via (at 143.4211 92.3036) (size 1.016) (drill 0.508) (layers "F.Cu" "B.Cu") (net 4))
 (via (at 140.8811 92.3036) (size 1.016) (drill 0.508) (layers "F.Cu" "B.Cu") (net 4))
 (via (at 138.3411 92.3036) (size 1.016) (drill 0.508) (layers "F.Cu" "B.Cu") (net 4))
 (via (at 138.3411 122.7836) (size 1.016) (drill 0.508) (layers "F.Cu" "B.Cu") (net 4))
 (via (at 143.4211 122.7836) (size 1.016) (drill 0.508) (layers "F.Cu" "B.Cu") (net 4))
 (via (at 138.3411 112.6236) (size 1.016) (drill 0.508) (layers "F.Cu" "B.Cu") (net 4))
 (via (at 142.1511 117.7036) (size 1.016) (drill 0.508) (layers "F.Cu" "B.Cu") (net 4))
 (via (at 138.3411 102.4636) (size 1.016) (drill 0.508) (layers "F.Cu" "B.Cu") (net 4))
 (via (at 139.6111 107.5436) (size 1.016) (drill 0.508) (layers "F.Cu" "B.Cu") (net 4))
 (via (at 140.8811 112.6236) (size 1.016) (drill 0.508) (layers "F.Cu" "B.Cu") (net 4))
 (via (at 139.6111 127.8636) (size 1.016) (drill 0.508) (layers "F.Cu" "B.Cu") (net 4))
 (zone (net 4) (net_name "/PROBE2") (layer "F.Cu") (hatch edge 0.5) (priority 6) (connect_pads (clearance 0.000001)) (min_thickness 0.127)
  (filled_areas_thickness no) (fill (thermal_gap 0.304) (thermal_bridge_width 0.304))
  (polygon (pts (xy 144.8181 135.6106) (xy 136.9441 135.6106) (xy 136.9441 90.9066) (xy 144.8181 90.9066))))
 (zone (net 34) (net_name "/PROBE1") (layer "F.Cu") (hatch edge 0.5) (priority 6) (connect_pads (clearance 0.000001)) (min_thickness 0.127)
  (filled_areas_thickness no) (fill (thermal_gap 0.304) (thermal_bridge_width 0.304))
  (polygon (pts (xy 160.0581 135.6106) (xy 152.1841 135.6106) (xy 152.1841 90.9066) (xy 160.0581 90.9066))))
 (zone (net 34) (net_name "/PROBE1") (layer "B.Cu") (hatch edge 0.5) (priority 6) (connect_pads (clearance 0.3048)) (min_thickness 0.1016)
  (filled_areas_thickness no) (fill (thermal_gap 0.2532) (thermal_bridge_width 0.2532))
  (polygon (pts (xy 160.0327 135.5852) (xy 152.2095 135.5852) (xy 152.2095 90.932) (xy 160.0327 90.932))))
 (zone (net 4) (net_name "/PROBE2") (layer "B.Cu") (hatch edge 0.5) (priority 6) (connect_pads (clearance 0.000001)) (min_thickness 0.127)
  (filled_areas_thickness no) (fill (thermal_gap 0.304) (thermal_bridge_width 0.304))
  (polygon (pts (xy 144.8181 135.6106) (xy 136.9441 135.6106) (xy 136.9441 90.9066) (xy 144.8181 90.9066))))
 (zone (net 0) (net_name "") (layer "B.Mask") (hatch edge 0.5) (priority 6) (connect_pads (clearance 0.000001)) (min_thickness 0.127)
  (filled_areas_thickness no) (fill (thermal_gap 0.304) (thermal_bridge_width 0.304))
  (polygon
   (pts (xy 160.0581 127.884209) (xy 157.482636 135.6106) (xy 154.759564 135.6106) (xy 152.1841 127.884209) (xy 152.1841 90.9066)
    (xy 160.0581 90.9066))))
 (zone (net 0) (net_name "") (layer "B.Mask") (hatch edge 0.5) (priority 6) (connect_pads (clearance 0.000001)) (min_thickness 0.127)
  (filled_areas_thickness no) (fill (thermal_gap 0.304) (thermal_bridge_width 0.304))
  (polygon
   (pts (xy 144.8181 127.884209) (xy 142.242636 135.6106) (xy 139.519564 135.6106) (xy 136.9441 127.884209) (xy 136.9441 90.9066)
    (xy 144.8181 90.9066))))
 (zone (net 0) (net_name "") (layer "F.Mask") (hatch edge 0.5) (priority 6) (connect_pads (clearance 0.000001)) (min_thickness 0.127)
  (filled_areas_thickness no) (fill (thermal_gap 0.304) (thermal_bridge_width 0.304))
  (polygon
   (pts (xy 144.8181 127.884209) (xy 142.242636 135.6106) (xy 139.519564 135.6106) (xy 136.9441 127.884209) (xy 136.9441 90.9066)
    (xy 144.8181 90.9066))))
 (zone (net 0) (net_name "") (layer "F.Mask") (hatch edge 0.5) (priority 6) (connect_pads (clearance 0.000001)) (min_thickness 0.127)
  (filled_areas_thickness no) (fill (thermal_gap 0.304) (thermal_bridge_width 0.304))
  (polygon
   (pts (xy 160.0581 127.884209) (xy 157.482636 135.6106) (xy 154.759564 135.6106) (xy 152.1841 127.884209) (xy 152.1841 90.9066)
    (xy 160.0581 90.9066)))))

